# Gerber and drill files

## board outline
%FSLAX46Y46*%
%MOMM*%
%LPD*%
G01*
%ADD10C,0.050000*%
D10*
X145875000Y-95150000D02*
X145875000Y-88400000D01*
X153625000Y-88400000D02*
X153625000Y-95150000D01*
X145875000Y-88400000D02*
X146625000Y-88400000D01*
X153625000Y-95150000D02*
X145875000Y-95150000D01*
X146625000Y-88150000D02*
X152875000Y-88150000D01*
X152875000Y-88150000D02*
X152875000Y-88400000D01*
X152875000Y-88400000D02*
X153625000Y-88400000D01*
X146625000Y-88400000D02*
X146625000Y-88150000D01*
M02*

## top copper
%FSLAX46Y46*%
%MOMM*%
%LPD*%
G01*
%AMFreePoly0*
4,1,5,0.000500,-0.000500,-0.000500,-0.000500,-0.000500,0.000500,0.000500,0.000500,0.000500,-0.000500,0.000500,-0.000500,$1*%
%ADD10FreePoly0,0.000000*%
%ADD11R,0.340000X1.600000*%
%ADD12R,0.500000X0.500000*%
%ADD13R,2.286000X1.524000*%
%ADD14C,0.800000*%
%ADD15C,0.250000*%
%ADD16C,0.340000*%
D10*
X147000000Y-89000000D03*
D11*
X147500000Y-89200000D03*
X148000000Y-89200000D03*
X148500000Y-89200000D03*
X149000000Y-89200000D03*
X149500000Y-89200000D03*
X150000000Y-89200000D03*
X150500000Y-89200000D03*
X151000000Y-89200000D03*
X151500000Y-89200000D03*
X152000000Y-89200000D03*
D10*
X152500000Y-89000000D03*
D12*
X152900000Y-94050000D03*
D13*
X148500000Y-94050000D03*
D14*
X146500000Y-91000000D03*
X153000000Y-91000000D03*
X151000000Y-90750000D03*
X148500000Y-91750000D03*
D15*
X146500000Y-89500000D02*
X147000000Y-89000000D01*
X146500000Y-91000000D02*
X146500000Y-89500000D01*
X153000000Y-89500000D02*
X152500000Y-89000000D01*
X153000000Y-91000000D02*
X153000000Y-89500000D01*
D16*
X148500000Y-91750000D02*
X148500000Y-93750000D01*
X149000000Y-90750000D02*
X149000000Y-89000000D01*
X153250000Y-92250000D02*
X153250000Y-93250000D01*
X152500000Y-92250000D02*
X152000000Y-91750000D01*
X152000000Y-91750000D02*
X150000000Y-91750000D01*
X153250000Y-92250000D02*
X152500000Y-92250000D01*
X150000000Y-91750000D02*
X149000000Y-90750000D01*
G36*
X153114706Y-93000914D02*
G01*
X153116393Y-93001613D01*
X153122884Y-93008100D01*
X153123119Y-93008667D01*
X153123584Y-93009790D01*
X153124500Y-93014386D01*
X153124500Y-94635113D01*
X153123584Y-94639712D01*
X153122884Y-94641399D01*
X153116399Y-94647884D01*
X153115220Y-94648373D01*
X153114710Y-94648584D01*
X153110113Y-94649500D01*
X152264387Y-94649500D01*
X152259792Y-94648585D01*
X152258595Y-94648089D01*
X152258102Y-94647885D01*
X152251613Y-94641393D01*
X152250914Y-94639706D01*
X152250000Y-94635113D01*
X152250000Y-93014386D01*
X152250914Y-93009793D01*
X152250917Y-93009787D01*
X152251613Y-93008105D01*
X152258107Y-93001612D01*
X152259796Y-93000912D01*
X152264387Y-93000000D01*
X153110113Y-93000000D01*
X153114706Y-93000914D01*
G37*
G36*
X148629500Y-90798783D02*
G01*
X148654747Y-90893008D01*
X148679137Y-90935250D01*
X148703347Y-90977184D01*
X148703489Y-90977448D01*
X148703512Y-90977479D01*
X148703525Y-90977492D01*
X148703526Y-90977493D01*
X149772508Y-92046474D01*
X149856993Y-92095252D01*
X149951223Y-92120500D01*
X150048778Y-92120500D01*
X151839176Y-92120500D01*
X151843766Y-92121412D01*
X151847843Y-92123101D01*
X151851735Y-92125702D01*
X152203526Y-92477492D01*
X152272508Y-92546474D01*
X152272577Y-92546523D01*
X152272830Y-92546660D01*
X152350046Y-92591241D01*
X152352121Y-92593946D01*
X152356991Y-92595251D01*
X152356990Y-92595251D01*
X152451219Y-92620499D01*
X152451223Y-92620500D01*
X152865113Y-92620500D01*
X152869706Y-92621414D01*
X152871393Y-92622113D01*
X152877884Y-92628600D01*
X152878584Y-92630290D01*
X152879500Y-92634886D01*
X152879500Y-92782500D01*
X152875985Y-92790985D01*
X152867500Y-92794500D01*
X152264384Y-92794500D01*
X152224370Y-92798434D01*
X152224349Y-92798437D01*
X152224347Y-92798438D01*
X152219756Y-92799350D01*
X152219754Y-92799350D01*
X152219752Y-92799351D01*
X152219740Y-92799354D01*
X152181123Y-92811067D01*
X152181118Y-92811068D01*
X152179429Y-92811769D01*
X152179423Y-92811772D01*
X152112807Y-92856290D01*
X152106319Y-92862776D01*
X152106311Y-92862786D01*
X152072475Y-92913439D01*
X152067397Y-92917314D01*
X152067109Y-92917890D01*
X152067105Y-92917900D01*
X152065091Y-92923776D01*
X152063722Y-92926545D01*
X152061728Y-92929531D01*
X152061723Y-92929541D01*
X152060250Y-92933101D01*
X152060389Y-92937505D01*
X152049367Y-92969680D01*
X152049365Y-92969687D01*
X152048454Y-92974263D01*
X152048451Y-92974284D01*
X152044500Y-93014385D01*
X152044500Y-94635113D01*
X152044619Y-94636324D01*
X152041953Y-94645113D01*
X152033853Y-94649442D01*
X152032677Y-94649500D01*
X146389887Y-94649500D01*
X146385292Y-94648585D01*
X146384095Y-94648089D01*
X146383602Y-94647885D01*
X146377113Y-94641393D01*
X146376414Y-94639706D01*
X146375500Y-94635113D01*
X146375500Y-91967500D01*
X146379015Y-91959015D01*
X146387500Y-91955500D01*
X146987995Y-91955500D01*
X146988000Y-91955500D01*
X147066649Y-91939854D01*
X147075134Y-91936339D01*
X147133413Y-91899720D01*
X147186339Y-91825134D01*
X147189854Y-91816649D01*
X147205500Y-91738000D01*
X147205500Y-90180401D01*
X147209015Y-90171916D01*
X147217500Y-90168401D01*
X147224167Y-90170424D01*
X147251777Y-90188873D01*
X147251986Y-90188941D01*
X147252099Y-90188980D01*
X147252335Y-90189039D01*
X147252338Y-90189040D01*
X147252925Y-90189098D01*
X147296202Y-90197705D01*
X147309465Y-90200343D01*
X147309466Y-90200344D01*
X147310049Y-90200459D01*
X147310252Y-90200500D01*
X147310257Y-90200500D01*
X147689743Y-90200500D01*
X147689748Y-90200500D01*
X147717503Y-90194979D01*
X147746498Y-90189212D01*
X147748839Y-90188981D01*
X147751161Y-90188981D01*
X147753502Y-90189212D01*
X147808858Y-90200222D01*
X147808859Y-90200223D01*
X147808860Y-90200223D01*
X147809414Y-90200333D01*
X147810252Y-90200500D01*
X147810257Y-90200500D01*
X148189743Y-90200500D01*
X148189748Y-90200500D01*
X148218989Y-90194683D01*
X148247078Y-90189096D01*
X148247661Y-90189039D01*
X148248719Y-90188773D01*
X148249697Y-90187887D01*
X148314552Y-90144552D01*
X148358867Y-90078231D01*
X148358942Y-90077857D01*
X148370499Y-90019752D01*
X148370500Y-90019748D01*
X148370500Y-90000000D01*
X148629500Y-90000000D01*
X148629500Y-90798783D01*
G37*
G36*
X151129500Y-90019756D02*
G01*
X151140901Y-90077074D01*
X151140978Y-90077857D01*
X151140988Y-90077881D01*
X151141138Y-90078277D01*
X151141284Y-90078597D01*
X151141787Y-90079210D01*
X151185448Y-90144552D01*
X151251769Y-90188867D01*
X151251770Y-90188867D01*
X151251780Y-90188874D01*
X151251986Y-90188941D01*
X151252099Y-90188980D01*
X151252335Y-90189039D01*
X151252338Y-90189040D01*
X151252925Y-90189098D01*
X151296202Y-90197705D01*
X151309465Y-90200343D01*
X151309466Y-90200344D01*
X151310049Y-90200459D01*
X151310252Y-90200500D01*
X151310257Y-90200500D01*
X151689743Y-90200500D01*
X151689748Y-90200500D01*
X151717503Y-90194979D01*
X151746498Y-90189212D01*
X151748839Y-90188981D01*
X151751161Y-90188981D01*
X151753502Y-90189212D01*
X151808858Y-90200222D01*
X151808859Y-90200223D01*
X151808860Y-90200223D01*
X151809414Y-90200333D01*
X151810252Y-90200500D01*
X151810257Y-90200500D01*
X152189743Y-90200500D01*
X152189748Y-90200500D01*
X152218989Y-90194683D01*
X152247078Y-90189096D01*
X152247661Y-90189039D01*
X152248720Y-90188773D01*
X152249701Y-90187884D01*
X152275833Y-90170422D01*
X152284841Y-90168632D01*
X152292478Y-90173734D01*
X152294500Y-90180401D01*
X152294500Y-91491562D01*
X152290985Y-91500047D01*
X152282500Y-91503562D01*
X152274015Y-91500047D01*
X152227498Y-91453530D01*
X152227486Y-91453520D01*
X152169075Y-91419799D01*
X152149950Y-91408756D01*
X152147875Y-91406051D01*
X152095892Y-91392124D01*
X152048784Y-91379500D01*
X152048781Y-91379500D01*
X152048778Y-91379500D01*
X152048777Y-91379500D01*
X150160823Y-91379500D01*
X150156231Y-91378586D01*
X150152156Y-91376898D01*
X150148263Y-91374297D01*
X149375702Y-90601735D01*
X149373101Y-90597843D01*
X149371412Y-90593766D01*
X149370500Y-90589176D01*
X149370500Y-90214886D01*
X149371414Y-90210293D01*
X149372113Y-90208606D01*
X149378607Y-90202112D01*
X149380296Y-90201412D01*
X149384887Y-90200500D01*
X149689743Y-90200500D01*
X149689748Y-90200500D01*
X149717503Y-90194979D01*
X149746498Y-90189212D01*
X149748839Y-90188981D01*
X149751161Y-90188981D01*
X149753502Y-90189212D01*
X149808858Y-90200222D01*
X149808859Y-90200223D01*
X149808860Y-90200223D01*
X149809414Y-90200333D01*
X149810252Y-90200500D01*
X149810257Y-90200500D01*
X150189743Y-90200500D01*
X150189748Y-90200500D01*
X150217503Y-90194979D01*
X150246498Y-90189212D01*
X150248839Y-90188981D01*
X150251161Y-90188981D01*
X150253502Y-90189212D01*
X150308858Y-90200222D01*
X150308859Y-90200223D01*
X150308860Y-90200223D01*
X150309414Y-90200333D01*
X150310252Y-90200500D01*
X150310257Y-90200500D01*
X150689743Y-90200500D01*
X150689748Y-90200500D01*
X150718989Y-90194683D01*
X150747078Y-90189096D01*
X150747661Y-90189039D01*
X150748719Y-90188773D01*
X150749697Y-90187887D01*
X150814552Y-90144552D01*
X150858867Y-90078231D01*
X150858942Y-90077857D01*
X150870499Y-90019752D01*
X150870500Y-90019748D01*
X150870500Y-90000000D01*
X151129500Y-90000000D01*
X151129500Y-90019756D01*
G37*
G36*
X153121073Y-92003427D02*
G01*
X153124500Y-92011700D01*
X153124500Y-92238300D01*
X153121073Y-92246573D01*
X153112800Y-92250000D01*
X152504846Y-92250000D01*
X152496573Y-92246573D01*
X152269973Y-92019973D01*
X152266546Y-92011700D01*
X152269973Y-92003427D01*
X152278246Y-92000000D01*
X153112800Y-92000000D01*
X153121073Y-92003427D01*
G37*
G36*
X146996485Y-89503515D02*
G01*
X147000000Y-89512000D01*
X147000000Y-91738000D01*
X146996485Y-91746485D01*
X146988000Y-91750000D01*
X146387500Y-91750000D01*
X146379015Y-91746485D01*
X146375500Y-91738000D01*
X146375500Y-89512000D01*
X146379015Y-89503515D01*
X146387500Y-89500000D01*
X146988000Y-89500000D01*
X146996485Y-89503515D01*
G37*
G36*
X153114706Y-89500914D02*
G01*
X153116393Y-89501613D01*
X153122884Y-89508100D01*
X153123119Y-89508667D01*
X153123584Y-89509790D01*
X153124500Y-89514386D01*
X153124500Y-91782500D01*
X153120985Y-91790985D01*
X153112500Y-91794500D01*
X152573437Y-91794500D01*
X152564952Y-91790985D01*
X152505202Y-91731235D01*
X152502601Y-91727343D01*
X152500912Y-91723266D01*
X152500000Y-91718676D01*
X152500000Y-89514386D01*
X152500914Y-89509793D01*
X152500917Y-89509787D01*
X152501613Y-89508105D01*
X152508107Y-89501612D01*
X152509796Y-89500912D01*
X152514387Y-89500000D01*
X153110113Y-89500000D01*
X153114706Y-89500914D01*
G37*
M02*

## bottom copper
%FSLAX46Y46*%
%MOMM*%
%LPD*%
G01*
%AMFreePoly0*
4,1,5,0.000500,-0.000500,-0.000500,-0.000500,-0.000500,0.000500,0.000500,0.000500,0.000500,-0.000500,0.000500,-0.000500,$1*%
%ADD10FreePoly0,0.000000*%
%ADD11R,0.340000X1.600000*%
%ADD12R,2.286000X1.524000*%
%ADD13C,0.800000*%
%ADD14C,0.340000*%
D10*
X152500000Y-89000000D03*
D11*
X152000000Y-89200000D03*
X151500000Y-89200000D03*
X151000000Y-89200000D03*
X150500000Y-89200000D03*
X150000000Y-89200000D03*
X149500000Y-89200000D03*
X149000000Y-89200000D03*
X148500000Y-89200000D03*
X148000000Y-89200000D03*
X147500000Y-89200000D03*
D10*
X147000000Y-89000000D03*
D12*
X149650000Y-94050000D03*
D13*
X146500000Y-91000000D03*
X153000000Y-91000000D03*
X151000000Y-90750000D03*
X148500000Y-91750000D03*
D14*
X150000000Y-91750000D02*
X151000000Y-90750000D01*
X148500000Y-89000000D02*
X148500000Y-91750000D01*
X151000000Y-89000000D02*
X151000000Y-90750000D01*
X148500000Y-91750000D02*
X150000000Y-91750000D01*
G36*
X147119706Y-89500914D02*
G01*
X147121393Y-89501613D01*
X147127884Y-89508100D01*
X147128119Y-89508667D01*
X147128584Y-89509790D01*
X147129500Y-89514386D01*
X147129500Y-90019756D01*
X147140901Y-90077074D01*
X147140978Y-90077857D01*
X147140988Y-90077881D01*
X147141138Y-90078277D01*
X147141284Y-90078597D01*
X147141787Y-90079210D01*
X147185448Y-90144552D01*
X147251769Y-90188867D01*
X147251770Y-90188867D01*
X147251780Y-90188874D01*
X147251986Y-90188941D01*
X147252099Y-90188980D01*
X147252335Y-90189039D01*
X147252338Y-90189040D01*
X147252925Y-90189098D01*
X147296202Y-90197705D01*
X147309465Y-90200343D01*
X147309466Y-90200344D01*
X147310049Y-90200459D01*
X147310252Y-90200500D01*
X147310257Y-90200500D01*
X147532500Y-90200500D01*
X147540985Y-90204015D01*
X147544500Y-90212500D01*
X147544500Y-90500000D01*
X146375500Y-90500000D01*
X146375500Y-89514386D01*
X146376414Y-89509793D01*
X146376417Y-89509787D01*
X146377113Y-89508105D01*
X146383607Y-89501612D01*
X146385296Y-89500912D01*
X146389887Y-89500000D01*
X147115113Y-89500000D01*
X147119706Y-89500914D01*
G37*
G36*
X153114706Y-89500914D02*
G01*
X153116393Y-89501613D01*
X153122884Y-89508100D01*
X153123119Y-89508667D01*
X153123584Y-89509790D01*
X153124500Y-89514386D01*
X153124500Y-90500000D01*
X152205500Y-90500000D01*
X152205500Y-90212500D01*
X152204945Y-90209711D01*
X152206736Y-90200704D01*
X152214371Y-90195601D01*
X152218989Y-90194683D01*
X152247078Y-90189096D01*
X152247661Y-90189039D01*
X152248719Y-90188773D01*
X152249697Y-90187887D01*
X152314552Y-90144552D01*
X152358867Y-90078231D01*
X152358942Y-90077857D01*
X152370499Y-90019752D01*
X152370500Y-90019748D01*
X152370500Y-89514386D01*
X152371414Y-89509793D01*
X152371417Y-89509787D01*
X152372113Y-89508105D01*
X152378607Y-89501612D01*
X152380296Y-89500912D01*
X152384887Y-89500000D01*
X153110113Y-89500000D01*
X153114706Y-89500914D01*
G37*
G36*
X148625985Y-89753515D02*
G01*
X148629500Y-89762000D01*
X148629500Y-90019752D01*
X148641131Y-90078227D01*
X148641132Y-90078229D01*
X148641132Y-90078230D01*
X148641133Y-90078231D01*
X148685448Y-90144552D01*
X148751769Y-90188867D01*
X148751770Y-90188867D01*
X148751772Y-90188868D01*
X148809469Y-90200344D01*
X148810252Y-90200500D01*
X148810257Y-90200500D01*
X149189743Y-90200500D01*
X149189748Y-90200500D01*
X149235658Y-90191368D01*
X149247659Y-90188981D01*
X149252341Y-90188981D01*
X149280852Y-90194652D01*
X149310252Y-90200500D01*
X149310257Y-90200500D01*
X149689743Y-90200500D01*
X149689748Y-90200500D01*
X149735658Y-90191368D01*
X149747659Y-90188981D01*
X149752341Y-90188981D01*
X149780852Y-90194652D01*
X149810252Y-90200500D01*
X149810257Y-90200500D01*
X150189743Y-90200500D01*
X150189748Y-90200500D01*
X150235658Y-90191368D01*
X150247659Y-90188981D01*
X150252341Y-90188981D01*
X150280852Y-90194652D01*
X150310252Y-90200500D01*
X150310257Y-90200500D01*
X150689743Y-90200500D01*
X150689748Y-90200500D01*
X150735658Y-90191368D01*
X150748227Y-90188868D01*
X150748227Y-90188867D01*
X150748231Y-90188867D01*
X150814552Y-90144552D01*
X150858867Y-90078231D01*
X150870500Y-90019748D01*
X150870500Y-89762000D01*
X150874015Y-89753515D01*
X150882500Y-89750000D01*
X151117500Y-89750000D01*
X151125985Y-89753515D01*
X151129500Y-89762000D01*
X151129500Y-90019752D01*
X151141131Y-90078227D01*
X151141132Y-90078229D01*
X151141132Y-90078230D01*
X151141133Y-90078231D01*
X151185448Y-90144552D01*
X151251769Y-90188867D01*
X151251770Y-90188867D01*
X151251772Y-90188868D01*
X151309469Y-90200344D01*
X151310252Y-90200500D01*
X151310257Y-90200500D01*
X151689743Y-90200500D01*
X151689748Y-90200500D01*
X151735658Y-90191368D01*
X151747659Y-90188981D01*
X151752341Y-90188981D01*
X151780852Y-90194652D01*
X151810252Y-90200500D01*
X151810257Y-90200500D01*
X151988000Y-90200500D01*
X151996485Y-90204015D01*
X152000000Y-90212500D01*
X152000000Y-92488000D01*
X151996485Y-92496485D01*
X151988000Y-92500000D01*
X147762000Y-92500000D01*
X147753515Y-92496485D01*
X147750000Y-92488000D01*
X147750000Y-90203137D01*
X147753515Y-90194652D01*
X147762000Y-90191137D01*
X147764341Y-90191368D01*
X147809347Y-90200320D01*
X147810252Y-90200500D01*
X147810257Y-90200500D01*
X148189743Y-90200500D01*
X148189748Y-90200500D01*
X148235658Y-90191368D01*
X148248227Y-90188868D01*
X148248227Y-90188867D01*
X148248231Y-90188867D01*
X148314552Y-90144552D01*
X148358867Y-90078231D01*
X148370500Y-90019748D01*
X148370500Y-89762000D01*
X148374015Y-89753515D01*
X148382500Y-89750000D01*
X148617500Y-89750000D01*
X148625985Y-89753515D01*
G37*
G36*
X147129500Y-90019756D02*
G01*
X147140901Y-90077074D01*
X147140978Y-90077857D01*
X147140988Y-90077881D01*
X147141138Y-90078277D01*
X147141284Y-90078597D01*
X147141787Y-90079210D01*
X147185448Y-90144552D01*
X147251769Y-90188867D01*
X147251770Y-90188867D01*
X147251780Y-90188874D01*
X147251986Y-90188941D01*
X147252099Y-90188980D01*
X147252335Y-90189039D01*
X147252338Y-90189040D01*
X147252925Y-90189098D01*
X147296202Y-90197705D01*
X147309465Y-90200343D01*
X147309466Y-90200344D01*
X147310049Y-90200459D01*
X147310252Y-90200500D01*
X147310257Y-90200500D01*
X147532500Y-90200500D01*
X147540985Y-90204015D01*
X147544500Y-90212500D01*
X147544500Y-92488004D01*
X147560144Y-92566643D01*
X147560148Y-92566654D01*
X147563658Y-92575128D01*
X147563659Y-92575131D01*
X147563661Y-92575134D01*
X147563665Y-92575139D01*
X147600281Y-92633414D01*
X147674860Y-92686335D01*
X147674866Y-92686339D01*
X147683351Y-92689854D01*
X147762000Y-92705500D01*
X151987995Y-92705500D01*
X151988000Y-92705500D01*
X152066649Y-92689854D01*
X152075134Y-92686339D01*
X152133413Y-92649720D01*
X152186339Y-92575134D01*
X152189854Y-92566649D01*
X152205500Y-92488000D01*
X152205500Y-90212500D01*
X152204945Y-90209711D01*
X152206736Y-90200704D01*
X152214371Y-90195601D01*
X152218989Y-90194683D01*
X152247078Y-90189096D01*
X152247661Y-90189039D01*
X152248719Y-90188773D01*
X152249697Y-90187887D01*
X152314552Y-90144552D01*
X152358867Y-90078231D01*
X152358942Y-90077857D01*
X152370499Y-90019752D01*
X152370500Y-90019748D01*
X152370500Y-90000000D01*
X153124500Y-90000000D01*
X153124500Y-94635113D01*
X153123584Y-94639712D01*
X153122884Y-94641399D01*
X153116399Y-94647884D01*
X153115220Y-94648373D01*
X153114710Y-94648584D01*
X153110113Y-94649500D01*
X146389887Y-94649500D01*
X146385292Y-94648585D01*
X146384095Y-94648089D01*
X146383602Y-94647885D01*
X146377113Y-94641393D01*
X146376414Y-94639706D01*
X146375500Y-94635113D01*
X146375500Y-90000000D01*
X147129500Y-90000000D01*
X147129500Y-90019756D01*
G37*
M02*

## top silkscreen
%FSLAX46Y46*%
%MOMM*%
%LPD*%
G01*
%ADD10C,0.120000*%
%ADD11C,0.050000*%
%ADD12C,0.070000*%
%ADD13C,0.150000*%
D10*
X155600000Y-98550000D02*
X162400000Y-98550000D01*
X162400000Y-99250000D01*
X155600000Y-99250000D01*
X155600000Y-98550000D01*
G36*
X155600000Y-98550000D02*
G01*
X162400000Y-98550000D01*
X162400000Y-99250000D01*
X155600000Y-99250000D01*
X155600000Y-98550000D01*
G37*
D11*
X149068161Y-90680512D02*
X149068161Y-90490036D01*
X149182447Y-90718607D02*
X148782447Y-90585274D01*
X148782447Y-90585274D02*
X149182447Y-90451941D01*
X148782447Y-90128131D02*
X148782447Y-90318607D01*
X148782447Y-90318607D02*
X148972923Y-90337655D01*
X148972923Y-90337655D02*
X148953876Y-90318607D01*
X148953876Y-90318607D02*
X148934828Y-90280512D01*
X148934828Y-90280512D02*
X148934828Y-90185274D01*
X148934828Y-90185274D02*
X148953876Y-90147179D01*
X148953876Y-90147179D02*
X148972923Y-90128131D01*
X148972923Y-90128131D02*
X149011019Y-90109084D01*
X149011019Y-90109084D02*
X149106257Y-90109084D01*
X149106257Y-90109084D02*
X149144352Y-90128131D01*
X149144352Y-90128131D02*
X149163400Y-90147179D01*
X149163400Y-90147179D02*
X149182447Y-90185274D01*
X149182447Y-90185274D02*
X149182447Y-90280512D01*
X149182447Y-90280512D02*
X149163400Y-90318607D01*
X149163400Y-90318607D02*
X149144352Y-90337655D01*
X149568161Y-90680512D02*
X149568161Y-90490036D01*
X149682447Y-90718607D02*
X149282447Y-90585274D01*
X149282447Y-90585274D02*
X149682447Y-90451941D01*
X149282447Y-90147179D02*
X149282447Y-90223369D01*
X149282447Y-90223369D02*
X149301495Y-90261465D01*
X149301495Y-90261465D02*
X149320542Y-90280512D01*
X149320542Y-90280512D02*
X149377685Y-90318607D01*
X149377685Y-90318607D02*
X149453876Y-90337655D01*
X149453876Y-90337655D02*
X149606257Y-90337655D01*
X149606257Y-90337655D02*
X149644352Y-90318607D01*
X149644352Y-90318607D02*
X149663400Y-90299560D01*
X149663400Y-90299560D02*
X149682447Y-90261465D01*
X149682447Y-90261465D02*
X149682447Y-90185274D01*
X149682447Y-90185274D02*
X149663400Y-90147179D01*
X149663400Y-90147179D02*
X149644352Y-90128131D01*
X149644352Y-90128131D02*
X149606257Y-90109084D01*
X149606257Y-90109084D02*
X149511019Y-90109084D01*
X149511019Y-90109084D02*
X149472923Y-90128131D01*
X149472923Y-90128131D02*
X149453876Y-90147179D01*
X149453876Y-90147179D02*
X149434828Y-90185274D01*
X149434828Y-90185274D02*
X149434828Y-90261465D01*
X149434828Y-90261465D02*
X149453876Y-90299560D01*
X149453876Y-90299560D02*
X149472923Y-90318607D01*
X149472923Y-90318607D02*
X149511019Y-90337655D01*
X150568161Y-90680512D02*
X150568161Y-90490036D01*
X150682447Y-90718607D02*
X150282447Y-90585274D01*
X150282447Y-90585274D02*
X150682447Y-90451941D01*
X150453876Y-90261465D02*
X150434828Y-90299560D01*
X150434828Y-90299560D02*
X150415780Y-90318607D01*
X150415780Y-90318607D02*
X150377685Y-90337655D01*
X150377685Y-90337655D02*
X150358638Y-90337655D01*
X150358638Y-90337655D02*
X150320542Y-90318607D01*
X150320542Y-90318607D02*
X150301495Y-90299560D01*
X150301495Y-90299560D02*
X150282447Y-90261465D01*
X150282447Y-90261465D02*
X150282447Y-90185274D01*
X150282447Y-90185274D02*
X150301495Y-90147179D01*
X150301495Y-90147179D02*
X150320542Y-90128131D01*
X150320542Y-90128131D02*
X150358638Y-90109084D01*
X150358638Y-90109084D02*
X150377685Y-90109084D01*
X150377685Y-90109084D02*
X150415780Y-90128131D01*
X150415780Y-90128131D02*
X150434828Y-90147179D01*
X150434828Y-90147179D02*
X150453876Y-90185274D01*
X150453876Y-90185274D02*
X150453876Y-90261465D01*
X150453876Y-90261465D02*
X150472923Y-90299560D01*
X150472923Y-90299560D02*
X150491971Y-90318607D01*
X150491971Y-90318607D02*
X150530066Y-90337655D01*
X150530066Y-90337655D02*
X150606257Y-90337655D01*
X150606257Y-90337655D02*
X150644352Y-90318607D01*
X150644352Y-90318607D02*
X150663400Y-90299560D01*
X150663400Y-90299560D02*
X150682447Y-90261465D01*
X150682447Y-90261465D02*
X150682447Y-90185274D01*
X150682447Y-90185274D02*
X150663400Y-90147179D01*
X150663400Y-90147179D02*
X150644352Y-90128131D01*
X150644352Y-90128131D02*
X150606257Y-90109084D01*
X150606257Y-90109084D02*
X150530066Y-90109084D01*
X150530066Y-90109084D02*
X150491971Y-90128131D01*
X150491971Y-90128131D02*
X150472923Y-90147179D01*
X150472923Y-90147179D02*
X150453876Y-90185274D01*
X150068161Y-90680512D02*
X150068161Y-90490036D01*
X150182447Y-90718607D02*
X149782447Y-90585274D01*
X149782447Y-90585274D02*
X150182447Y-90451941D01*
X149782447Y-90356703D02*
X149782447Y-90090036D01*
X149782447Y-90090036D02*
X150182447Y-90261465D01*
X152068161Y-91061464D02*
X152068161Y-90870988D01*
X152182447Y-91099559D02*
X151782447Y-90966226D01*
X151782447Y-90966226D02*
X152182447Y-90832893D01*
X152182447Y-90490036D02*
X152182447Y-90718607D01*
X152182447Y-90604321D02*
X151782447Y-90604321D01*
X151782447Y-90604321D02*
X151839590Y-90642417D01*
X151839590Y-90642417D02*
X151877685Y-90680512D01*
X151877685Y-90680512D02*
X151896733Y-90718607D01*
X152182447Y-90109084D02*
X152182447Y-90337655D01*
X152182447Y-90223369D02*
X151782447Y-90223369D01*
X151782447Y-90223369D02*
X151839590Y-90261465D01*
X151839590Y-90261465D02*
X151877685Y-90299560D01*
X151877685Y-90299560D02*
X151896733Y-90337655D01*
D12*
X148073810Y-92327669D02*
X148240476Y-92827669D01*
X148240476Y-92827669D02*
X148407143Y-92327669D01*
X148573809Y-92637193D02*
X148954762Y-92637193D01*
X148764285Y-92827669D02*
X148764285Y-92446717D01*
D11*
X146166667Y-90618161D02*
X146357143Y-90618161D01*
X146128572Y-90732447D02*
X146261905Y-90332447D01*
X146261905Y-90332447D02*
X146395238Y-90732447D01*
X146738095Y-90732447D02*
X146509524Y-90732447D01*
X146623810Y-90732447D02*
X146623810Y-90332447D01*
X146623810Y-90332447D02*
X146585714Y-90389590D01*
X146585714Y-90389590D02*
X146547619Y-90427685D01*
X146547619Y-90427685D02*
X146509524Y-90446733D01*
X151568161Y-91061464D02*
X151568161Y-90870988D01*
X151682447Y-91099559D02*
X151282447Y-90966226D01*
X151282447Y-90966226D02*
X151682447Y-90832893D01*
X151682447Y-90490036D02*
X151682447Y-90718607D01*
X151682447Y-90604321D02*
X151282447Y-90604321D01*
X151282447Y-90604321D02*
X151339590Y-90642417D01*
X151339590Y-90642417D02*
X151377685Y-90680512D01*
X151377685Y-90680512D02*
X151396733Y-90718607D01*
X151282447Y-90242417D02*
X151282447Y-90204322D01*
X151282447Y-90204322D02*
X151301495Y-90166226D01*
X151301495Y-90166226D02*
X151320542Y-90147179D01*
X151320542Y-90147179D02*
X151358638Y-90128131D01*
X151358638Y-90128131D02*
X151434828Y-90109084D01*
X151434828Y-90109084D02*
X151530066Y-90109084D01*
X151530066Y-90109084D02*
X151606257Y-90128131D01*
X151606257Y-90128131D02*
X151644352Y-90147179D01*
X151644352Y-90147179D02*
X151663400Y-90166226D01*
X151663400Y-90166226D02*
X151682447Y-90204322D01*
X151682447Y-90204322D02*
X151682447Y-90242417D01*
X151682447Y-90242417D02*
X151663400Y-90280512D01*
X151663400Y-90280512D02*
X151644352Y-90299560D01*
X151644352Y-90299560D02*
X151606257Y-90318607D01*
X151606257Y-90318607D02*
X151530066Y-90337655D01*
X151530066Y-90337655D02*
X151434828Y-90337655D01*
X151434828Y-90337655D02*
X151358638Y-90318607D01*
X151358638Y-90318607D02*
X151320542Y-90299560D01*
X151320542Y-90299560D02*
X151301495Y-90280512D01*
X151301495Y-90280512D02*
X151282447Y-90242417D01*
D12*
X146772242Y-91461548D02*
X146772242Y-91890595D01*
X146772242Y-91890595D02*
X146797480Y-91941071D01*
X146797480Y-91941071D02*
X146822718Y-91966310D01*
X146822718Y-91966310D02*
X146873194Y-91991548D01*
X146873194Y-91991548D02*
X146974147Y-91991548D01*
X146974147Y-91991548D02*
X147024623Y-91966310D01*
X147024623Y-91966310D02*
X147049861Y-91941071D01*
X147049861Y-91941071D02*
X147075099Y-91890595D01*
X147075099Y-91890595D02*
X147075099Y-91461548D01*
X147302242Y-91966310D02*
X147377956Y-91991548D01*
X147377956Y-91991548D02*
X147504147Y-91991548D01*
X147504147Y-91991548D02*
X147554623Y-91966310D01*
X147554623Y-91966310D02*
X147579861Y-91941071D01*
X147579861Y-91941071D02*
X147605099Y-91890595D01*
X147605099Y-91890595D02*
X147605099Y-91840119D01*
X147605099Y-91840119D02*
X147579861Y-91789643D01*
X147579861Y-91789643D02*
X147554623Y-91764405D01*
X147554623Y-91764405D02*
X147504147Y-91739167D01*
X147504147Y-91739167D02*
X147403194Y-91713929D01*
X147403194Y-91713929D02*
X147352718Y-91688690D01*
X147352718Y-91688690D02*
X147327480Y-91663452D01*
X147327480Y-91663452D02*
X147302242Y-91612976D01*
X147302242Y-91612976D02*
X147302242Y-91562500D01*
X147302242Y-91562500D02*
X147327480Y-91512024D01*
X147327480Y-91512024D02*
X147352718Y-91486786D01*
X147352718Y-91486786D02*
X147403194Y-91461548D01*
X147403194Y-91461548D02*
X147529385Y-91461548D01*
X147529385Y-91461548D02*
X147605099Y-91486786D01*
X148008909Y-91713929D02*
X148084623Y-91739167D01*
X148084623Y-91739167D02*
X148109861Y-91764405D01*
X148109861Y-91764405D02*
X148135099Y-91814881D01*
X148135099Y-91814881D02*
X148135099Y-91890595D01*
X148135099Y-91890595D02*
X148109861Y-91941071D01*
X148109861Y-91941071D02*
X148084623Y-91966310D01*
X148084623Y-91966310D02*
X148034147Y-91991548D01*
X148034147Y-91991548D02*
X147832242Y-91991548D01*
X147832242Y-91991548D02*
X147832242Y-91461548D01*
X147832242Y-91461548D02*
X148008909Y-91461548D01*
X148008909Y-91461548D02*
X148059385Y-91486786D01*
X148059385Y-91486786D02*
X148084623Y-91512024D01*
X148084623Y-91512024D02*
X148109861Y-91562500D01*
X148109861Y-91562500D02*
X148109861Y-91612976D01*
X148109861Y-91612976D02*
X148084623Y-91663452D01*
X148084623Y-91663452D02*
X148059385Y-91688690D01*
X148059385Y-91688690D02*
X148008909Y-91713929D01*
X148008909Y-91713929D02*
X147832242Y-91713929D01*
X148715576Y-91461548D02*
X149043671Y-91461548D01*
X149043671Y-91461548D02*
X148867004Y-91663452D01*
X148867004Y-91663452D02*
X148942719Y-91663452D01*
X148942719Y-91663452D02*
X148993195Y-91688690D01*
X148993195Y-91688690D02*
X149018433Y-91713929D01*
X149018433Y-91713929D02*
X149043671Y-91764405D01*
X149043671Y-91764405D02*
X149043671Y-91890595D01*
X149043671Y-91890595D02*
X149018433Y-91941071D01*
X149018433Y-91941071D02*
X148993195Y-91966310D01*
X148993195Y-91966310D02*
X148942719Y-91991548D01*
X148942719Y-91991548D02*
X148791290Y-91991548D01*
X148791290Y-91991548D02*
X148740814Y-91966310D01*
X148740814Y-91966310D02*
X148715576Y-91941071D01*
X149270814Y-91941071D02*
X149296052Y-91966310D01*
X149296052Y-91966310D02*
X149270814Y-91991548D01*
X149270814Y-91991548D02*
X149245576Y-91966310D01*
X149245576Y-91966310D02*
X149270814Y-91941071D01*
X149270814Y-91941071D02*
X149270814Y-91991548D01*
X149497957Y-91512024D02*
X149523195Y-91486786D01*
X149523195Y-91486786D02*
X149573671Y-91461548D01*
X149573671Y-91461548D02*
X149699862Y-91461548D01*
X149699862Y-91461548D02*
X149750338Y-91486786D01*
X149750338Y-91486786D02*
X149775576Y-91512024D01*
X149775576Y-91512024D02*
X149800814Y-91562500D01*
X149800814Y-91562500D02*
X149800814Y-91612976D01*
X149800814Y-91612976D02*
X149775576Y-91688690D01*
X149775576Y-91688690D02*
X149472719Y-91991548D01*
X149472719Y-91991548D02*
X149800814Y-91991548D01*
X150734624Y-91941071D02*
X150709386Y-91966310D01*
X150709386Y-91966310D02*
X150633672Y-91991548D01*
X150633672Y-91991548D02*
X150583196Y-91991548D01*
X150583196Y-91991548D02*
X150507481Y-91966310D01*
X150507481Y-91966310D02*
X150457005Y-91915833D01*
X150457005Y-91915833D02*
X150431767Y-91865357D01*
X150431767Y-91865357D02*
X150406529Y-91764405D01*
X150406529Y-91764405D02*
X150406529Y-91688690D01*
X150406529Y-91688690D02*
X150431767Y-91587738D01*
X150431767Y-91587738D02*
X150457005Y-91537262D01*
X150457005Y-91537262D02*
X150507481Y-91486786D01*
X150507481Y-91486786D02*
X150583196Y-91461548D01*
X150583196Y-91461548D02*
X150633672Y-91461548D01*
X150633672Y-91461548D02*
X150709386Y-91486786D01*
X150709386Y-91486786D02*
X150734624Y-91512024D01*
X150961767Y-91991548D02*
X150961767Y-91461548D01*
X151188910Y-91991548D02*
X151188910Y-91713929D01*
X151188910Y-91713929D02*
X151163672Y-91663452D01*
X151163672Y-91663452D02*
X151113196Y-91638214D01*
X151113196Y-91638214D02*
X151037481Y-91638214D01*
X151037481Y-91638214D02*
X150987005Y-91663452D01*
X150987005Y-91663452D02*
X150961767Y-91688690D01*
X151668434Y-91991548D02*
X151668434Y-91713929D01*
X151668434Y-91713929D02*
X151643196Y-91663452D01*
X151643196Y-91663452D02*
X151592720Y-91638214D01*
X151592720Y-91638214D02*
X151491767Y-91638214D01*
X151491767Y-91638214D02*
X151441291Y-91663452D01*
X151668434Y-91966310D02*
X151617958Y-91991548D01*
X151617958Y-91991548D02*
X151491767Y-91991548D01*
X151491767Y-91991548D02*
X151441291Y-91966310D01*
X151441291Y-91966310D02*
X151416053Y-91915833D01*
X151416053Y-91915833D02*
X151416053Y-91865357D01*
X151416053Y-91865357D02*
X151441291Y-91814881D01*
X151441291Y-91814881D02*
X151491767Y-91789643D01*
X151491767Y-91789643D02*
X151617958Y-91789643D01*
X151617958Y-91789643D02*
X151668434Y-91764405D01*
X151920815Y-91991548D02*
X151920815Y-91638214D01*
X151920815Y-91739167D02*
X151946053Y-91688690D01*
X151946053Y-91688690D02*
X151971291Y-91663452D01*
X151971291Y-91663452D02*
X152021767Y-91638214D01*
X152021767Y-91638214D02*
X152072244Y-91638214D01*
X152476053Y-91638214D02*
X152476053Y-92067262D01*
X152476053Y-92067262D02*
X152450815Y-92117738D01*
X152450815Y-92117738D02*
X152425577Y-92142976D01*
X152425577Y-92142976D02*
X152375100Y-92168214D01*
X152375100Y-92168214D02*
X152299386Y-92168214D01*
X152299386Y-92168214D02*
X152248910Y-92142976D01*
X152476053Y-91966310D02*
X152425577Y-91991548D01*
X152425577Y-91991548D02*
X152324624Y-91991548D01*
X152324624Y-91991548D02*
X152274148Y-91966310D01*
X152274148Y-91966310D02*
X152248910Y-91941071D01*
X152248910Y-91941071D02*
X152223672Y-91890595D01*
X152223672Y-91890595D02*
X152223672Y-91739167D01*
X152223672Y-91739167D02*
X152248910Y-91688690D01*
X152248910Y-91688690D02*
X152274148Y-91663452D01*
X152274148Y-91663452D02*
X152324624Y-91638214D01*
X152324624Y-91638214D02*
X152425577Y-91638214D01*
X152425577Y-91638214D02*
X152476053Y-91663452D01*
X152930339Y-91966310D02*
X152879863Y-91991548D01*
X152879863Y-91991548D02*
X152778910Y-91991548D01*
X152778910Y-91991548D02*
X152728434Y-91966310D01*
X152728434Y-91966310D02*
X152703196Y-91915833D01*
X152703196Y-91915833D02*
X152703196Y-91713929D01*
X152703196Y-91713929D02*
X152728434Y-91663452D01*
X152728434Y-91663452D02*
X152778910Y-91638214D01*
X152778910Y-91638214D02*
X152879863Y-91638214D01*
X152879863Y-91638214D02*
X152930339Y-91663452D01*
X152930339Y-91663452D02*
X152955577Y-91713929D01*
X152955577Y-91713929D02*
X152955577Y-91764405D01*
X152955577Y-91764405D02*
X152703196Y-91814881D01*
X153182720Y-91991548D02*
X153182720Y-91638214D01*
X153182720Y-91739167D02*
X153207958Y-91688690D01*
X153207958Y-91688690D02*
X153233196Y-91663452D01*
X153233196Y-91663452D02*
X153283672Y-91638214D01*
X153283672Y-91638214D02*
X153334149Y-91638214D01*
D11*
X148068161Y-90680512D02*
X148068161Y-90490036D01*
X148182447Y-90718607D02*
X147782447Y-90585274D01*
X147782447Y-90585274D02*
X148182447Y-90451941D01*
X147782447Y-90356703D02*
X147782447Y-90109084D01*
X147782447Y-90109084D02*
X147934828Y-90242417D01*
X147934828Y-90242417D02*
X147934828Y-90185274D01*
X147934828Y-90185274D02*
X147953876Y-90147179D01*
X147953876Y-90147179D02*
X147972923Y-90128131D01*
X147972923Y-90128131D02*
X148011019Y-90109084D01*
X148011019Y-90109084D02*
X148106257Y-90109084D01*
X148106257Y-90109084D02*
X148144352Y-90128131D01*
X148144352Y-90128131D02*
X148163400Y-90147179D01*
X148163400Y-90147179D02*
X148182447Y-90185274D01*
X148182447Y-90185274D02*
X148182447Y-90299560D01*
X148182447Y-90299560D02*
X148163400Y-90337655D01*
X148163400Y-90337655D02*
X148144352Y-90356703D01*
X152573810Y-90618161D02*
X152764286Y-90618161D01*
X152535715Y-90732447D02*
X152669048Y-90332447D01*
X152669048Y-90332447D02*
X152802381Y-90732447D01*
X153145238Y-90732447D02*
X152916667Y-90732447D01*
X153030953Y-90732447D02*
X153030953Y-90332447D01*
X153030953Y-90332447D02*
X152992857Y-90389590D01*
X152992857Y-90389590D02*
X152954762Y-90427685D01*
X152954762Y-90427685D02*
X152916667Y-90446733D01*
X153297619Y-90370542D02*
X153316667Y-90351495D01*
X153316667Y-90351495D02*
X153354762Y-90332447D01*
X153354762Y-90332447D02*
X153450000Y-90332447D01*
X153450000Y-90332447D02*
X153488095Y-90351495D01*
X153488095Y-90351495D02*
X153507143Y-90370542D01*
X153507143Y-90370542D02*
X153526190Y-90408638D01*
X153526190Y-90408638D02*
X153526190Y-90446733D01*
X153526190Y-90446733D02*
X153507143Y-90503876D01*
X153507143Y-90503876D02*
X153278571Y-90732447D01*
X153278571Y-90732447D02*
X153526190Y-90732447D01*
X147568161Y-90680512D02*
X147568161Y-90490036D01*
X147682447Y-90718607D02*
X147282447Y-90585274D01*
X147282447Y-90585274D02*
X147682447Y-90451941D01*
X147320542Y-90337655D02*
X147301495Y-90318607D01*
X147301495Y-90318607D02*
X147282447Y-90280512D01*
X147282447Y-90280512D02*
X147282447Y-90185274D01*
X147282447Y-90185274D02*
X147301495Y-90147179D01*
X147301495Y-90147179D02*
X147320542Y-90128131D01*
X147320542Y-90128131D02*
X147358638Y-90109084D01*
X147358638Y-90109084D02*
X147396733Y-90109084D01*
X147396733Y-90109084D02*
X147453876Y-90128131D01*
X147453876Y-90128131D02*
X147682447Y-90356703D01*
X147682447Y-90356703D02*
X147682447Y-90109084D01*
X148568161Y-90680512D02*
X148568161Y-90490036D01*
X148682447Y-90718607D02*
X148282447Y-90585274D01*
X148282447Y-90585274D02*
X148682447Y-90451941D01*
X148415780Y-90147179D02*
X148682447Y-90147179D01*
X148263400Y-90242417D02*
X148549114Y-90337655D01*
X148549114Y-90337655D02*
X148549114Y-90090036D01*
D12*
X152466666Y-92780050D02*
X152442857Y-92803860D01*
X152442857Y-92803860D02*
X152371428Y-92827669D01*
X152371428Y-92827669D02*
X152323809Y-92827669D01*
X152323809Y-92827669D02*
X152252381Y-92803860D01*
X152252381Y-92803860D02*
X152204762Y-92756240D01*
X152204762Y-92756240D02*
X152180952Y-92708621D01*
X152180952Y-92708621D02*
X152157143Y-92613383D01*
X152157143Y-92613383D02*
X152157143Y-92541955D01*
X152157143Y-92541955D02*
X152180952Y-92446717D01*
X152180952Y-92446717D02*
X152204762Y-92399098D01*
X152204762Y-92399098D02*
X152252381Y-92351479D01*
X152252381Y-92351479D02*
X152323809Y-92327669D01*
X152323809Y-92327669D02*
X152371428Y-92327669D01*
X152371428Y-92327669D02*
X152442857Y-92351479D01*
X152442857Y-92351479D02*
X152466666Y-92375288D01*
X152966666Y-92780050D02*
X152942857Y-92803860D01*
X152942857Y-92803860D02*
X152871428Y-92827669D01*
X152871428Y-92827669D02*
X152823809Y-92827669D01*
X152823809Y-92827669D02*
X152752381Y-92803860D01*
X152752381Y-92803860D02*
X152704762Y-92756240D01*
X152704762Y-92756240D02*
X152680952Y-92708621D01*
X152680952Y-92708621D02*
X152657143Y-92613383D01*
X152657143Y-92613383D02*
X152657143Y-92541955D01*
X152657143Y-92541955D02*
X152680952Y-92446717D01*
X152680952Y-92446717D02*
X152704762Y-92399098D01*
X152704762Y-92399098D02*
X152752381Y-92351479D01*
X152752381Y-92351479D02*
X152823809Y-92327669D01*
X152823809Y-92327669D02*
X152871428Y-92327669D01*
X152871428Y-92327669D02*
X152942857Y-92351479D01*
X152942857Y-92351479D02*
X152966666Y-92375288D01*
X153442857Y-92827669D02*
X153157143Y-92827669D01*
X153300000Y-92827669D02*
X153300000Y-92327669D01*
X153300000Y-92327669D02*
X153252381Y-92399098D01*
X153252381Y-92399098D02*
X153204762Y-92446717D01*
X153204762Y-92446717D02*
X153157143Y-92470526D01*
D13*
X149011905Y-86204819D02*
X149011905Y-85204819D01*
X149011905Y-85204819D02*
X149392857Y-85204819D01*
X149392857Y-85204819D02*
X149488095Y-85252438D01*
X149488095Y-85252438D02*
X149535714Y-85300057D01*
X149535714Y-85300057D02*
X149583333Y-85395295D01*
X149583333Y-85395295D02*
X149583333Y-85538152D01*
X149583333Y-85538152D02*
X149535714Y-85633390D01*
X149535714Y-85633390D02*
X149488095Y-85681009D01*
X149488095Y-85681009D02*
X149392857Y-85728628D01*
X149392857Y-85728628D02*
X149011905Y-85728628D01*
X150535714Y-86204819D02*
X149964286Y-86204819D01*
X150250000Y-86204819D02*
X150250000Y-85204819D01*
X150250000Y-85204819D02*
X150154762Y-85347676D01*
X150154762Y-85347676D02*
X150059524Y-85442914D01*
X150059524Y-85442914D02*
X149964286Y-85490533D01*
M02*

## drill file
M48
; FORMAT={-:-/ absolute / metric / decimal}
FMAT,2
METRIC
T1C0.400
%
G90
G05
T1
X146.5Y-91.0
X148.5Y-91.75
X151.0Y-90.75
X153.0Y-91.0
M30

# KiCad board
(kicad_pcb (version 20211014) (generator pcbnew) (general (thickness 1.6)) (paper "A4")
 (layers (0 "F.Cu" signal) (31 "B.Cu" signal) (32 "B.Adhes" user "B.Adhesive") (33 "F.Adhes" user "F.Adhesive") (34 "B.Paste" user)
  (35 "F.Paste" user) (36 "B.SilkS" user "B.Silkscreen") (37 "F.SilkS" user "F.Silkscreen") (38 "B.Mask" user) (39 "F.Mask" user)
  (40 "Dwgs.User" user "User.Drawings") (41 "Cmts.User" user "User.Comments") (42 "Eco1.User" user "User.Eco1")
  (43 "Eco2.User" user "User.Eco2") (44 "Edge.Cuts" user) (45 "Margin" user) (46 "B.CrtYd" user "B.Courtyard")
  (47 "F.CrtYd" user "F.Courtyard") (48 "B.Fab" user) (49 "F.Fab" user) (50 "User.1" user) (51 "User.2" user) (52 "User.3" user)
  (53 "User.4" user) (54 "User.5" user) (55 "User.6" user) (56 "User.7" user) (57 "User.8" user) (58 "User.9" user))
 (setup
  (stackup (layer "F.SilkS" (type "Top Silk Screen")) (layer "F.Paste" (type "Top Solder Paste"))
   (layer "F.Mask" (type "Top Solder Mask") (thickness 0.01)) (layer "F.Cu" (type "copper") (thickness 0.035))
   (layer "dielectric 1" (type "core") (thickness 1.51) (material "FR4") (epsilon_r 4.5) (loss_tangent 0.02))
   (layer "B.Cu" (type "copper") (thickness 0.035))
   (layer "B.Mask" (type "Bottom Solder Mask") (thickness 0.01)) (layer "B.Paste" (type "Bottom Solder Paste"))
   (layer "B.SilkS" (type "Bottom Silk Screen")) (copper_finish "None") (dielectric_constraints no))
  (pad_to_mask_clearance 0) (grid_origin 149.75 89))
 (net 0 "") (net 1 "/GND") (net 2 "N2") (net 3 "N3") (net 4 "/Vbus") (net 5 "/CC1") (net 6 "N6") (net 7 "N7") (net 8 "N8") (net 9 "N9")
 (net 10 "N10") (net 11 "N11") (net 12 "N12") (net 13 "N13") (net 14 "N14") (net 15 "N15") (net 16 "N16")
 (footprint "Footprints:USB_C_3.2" (layer "F.Cu") (at 149.75 89)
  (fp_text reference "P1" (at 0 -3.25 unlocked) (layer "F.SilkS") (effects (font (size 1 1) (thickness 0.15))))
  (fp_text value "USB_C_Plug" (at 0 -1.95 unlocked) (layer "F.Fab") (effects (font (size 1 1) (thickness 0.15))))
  (pad "A1" smd custom (at -2.75 0) (size 0.001 0.001) (layers "F.Cu" "F.Paste" "F.Mask") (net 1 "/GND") (solder_mask_margin 0.1)
   (zone_connect 2) (options (clearance outline) (anchor rect)) (primitives))
  (pad "A2" smd rect (at -2.25 0.2) (size 0.34 1.6) (layers "F.Cu" "F.Paste" "F.Mask") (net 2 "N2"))
  (pad "A3" smd rect (at -1.75 0.2) (size 0.34 1.6) (layers "F.Cu" "F.Paste" "F.Mask") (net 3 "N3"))
  (pad "A4" smd rect (at -1.25 0.2) (size 0.34 1.6) (layers "F.Cu" "F.Paste" "F.Mask") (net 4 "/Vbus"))
  (pad "A5" smd rect (at -0.75 0.2) (size 0.34 1.6) (layers "F.Cu" "F.Paste" "F.Mask") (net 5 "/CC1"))
  (pad "A6" smd rect (at -0.25 0.2) (size 0.34 1.6) (layers "F.Cu" "F.Paste" "F.Mask") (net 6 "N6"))
  (pad "A7" smd rect (at 0.25 0.2) (size 0.34 1.6) (layers "F.Cu" "F.Paste" "F.Mask") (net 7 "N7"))
  (pad "A8" smd rect (at 0.75 0.2) (size 0.34 1.6) (layers "F.Cu" "F.Paste" "F.Mask") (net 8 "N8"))
  (pad "A9" smd rect (at 1.25 0.2) (size 0.34 1.6) (layers "F.Cu" "F.Paste" "F.Mask") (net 4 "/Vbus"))
  (pad "A10" smd rect (at 1.75 0.2) (size 0.34 1.6) (layers "F.Cu" "F.Paste" "F.Mask") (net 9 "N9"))
  (pad "A11" smd rect (at 2.25 0.2) (size 0.34 1.6) (layers "F.Cu" "F.Paste" "F.Mask") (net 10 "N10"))
  (pad "A12" smd custom (at 2.75 0) (size 0.001 0.001) (layers "F.Cu" "F.Paste" "F.Mask") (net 1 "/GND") (solder_mask_margin 0.1)
   (zone_connect 2) (options (clearance outline) (anchor rect)) (primitives))
  (pad "B1" smd custom (at 2.75 0) (size 0.001 0.001) (layers "B.Cu" "B.Paste" "B.Mask") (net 1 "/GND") (solder_mask_margin 0.1)
   (zone_connect 2) (options (clearance outline) (anchor rect)) (primitives))
  (pad "B2" smd rect (at 2.25 0.2) (size 0.34 1.6) (layers "B.Cu" "B.Paste" "B.Mask") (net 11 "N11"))
  (pad "B3" smd rect (at 1.75 0.2) (size 0.34 1.6) (layers "B.Cu" "B.Paste" "B.Mask") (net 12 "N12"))
  (pad "B4" smd rect (at 1.25 0.2) (size 0.34 1.6) (layers "B.Cu" "B.Paste" "B.Mask") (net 4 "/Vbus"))
  (pad "B5" smd rect (at 0.75 0.2) (size 0.34 1.6) (layers "B.Cu" "B.Paste" "B.Mask") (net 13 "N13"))
  (pad "B6" smd rect (at 0.25 0.2) (size 0.34 1.6) (layers "B.Cu" "B.Paste" "B.Mask"))
  (pad "B7" smd rect (at -0.25 0.2) (size 0.34 1.6) (layers "B.Cu" "B.Paste" "B.Mask"))
  (pad "B8" smd rect (at -0.75 0.2) (size 0.34 1.6) (layers "B.Cu" "B.Paste" "B.Mask") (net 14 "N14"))
  (pad "B9" smd rect (at -1.25 0.2) (size 0.34 1.6) (layers "B.Cu" "B.Paste" "B.Mask") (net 4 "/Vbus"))
  (pad "B10" smd rect (at -1.75 0.2) (size 0.34 1.6) (layers "B.Cu" "B.Paste" "B.Mask") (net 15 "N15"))
  (pad "B11" smd rect (at -2.25 0.2) (size 0.34 1.6) (layers "B.Cu" "B.Paste" "B.Mask") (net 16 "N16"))
  (pad "B12" smd custom (at -2.75 0) (size 0.001 0.001) (layers "B.Cu" "B.Paste" "B.Mask") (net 1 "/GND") (solder_mask_margin 0.1)
   (zone_connect 2) (options (clearance outline) (anchor rect)) (primitives)))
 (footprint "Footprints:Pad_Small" (layer "F.Cu") (at 152.9 94.05)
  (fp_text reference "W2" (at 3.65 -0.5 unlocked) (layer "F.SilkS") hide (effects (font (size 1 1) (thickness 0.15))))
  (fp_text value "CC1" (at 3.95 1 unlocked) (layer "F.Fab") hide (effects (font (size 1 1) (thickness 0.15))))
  (pad "1" smd rect (at 0 0) (size 0.5 0.5) (layers "F.Cu" "F.Paste" "F.Mask") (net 5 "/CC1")))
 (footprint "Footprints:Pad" (layer "F.Cu") (at 148.5 94.05)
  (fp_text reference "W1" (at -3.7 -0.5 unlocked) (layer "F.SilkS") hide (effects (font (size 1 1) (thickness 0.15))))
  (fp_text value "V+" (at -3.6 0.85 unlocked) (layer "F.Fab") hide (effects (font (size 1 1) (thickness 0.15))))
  (pad "1" smd rect (at 0 0) (size 2.286 1.524) (layers "F.Cu" "F.Paste" "F.Mask") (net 4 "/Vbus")))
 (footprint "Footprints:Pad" (layer "B.Cu") (at 149.65 94.05 180)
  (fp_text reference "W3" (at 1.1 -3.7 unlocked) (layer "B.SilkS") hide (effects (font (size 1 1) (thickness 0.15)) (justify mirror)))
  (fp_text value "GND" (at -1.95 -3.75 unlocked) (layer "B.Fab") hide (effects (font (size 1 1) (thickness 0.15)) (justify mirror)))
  (pad "1" smd rect (at 0 0 180) (size 2.286 1.524) (layers "B.Cu" "B.Paste" "B.Mask") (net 1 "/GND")))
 (gr_rect (start 155.6 99.25) (end 162.4 98.55) (layer "F.SilkS") (width 0.12) (fill solid))
 (gr_line (start 145.875 95.15) (end 145.875 88.4) (layer "Edge.Cuts") (width 0.05))
 (gr_line (start 153.625 88.4) (end 153.625 95.15) (layer "Edge.Cuts") (width 0.05))
 (gr_line (start 145.875 88.4) (end 146.625 88.4) (layer "Edge.Cuts") (width 0.05))
 (gr_line (start 153.625 95.15) (end 145.875 95.15) (layer "Edge.Cuts") (width 0.05))
 (gr_line (start 146.625 88.15) (end 152.875 88.15) (layer "Edge.Cuts") (width 0.05))
 (gr_line (start 152.875 88.15) (end 152.875 88.4) (layer "Edge.Cuts") (width 0.05))
 (gr_line (start 152.875 88.4) (end 153.625 88.4) (layer "Edge.Cuts") (width 0.05))
 (gr_line (start 146.625 88.4) (end 146.625 88.15) (layer "Edge.Cuts") (width 0.05))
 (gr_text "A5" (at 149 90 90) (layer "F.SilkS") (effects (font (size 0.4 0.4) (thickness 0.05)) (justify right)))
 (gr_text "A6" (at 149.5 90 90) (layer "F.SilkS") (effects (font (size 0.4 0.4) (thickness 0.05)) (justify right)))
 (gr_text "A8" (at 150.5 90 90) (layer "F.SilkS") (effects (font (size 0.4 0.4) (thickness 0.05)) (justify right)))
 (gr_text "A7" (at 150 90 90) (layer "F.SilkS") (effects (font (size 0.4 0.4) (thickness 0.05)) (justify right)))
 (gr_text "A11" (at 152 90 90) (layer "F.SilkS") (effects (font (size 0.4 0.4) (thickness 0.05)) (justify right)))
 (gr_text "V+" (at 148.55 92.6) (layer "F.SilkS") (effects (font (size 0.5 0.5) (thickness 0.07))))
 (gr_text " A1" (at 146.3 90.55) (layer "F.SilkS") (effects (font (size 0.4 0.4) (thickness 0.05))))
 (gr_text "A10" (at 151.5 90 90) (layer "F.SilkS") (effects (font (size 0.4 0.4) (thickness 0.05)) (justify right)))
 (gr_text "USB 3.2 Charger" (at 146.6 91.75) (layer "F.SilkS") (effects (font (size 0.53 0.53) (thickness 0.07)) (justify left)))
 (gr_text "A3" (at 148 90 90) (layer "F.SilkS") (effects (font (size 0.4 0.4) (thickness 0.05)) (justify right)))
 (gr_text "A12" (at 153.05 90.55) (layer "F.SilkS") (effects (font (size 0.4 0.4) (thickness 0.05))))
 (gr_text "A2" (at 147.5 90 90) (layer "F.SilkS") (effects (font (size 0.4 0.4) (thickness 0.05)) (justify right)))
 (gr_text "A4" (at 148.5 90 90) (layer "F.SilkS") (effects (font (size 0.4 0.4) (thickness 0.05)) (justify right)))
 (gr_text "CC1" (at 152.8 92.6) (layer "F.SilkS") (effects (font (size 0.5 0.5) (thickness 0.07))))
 (segment (start 146.5 89.5) (end 147 89) (width 0.25) (layer "F.Cu") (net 1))
 (segment (start 146.5 91) (end 146.5 89.5) (width 0.25) (layer "F.Cu") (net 1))
 (segment (start 153 89.5) (end 152.5 89) (width 0.25) (layer "F.Cu") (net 1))
 (segment (start 153 91) (end 153 89.5) (width 0.25) (layer "F.Cu") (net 1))
 (via (at 146.5 91) (size 0.8) (drill 0.4) (layers "F.Cu" "B.Cu") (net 1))
 (via (at 153 91) (size 0.8) (drill 0.4) (layers "F.Cu" "B.Cu") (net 1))
 (segment (start 148.5 91.75) (end 148.5 93.75) (width 0.34) (layer "F.Cu") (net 4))
 (via (at 151 90.75) (size 0.8) (drill 0.4) (layers "F.Cu" "B.Cu") (free) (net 4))
 (via (at 148.5 91.75) (size 0.8) (drill 0.4) (layers "F.Cu" "B.Cu") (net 4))
 (segment (start 150 91.75) (end 151 90.75) (width 0.34) (layer "B.Cu") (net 4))
 (segment (start 148.5 89) (end 148.5 91.75) (width 0.34) (layer "B.Cu") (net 4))
 (segment (start 151 89) (end 151 90.75) (width 0.34) (layer "B.Cu") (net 4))
 (segment (start 148.5 91.75) (end 150 91.75) (width 0.34) (layer "B.Cu") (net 4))
 (segment (start 149 90.75) (end 149 89) (width 0.34) (layer "F.Cu") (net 5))
 (segment (start 153.25 92.25) (end 153.25 93.25) (width 0.34) (layer "F.Cu") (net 5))
 (segment (start 152.5 92.25) (end 152 91.75) (width 0.34) (layer "F.Cu") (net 5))
 (segment (start 152 91.75) (end 150 91.75) (width 0.34) (layer "F.Cu") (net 5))
 (segment (start 153.25 92.25) (end 152.5 92.25) (width 0.34) (layer "F.Cu") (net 5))
 (segment (start 150 91.75) (end 149 90.75) (width 0.34) (layer "F.Cu") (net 5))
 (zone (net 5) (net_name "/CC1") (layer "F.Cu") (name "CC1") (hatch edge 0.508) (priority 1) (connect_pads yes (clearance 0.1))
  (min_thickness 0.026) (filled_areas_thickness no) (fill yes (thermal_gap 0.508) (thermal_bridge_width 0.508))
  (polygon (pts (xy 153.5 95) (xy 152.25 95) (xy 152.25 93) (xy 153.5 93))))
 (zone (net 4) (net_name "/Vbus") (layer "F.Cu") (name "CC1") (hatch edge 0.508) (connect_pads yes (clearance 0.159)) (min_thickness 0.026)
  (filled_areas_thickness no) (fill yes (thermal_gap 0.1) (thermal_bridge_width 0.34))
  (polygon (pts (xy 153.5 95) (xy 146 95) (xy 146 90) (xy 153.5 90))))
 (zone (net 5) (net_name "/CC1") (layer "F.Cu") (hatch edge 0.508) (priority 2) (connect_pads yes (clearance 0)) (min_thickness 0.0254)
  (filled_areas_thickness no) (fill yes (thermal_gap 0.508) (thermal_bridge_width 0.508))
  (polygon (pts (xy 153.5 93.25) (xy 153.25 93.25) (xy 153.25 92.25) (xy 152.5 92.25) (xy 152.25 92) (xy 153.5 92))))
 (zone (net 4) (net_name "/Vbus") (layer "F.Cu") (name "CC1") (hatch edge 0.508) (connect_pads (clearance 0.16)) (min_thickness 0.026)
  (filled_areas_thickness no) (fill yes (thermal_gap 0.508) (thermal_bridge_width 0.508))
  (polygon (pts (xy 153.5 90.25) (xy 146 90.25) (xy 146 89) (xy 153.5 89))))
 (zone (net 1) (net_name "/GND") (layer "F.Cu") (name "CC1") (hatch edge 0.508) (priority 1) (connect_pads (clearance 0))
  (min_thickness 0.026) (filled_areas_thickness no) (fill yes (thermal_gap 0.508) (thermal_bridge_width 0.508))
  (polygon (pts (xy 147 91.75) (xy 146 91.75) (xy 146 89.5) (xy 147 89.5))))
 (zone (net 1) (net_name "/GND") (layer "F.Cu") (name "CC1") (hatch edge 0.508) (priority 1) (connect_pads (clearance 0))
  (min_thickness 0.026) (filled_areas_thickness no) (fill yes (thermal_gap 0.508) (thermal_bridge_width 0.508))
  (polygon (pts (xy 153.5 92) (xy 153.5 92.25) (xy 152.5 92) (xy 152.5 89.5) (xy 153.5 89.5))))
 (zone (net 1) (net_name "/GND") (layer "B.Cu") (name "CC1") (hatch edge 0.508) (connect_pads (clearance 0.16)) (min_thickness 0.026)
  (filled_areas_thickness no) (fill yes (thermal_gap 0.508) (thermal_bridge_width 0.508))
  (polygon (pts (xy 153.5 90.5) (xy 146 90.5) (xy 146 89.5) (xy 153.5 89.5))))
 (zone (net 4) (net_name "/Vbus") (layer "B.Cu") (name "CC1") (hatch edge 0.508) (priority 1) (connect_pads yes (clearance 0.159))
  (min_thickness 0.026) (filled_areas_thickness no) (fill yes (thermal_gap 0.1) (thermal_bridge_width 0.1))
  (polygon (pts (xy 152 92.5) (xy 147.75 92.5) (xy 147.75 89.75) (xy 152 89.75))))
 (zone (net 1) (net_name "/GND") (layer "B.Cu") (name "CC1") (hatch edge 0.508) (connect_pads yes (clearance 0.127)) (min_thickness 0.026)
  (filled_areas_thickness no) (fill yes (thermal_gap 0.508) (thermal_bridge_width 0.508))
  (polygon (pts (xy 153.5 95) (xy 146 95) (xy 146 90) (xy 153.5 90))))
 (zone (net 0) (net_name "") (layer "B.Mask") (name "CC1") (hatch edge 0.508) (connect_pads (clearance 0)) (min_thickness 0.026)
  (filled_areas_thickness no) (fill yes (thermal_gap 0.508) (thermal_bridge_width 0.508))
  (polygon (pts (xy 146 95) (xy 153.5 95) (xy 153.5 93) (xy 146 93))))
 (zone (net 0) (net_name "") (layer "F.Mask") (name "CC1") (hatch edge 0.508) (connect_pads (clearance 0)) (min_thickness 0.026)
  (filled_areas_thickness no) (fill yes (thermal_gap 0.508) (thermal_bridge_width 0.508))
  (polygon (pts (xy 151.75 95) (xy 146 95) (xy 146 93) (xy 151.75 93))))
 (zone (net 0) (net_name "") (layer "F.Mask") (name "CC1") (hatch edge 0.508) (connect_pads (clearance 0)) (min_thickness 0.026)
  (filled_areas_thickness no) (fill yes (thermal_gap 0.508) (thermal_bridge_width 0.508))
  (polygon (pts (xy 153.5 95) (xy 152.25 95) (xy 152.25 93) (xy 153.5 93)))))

